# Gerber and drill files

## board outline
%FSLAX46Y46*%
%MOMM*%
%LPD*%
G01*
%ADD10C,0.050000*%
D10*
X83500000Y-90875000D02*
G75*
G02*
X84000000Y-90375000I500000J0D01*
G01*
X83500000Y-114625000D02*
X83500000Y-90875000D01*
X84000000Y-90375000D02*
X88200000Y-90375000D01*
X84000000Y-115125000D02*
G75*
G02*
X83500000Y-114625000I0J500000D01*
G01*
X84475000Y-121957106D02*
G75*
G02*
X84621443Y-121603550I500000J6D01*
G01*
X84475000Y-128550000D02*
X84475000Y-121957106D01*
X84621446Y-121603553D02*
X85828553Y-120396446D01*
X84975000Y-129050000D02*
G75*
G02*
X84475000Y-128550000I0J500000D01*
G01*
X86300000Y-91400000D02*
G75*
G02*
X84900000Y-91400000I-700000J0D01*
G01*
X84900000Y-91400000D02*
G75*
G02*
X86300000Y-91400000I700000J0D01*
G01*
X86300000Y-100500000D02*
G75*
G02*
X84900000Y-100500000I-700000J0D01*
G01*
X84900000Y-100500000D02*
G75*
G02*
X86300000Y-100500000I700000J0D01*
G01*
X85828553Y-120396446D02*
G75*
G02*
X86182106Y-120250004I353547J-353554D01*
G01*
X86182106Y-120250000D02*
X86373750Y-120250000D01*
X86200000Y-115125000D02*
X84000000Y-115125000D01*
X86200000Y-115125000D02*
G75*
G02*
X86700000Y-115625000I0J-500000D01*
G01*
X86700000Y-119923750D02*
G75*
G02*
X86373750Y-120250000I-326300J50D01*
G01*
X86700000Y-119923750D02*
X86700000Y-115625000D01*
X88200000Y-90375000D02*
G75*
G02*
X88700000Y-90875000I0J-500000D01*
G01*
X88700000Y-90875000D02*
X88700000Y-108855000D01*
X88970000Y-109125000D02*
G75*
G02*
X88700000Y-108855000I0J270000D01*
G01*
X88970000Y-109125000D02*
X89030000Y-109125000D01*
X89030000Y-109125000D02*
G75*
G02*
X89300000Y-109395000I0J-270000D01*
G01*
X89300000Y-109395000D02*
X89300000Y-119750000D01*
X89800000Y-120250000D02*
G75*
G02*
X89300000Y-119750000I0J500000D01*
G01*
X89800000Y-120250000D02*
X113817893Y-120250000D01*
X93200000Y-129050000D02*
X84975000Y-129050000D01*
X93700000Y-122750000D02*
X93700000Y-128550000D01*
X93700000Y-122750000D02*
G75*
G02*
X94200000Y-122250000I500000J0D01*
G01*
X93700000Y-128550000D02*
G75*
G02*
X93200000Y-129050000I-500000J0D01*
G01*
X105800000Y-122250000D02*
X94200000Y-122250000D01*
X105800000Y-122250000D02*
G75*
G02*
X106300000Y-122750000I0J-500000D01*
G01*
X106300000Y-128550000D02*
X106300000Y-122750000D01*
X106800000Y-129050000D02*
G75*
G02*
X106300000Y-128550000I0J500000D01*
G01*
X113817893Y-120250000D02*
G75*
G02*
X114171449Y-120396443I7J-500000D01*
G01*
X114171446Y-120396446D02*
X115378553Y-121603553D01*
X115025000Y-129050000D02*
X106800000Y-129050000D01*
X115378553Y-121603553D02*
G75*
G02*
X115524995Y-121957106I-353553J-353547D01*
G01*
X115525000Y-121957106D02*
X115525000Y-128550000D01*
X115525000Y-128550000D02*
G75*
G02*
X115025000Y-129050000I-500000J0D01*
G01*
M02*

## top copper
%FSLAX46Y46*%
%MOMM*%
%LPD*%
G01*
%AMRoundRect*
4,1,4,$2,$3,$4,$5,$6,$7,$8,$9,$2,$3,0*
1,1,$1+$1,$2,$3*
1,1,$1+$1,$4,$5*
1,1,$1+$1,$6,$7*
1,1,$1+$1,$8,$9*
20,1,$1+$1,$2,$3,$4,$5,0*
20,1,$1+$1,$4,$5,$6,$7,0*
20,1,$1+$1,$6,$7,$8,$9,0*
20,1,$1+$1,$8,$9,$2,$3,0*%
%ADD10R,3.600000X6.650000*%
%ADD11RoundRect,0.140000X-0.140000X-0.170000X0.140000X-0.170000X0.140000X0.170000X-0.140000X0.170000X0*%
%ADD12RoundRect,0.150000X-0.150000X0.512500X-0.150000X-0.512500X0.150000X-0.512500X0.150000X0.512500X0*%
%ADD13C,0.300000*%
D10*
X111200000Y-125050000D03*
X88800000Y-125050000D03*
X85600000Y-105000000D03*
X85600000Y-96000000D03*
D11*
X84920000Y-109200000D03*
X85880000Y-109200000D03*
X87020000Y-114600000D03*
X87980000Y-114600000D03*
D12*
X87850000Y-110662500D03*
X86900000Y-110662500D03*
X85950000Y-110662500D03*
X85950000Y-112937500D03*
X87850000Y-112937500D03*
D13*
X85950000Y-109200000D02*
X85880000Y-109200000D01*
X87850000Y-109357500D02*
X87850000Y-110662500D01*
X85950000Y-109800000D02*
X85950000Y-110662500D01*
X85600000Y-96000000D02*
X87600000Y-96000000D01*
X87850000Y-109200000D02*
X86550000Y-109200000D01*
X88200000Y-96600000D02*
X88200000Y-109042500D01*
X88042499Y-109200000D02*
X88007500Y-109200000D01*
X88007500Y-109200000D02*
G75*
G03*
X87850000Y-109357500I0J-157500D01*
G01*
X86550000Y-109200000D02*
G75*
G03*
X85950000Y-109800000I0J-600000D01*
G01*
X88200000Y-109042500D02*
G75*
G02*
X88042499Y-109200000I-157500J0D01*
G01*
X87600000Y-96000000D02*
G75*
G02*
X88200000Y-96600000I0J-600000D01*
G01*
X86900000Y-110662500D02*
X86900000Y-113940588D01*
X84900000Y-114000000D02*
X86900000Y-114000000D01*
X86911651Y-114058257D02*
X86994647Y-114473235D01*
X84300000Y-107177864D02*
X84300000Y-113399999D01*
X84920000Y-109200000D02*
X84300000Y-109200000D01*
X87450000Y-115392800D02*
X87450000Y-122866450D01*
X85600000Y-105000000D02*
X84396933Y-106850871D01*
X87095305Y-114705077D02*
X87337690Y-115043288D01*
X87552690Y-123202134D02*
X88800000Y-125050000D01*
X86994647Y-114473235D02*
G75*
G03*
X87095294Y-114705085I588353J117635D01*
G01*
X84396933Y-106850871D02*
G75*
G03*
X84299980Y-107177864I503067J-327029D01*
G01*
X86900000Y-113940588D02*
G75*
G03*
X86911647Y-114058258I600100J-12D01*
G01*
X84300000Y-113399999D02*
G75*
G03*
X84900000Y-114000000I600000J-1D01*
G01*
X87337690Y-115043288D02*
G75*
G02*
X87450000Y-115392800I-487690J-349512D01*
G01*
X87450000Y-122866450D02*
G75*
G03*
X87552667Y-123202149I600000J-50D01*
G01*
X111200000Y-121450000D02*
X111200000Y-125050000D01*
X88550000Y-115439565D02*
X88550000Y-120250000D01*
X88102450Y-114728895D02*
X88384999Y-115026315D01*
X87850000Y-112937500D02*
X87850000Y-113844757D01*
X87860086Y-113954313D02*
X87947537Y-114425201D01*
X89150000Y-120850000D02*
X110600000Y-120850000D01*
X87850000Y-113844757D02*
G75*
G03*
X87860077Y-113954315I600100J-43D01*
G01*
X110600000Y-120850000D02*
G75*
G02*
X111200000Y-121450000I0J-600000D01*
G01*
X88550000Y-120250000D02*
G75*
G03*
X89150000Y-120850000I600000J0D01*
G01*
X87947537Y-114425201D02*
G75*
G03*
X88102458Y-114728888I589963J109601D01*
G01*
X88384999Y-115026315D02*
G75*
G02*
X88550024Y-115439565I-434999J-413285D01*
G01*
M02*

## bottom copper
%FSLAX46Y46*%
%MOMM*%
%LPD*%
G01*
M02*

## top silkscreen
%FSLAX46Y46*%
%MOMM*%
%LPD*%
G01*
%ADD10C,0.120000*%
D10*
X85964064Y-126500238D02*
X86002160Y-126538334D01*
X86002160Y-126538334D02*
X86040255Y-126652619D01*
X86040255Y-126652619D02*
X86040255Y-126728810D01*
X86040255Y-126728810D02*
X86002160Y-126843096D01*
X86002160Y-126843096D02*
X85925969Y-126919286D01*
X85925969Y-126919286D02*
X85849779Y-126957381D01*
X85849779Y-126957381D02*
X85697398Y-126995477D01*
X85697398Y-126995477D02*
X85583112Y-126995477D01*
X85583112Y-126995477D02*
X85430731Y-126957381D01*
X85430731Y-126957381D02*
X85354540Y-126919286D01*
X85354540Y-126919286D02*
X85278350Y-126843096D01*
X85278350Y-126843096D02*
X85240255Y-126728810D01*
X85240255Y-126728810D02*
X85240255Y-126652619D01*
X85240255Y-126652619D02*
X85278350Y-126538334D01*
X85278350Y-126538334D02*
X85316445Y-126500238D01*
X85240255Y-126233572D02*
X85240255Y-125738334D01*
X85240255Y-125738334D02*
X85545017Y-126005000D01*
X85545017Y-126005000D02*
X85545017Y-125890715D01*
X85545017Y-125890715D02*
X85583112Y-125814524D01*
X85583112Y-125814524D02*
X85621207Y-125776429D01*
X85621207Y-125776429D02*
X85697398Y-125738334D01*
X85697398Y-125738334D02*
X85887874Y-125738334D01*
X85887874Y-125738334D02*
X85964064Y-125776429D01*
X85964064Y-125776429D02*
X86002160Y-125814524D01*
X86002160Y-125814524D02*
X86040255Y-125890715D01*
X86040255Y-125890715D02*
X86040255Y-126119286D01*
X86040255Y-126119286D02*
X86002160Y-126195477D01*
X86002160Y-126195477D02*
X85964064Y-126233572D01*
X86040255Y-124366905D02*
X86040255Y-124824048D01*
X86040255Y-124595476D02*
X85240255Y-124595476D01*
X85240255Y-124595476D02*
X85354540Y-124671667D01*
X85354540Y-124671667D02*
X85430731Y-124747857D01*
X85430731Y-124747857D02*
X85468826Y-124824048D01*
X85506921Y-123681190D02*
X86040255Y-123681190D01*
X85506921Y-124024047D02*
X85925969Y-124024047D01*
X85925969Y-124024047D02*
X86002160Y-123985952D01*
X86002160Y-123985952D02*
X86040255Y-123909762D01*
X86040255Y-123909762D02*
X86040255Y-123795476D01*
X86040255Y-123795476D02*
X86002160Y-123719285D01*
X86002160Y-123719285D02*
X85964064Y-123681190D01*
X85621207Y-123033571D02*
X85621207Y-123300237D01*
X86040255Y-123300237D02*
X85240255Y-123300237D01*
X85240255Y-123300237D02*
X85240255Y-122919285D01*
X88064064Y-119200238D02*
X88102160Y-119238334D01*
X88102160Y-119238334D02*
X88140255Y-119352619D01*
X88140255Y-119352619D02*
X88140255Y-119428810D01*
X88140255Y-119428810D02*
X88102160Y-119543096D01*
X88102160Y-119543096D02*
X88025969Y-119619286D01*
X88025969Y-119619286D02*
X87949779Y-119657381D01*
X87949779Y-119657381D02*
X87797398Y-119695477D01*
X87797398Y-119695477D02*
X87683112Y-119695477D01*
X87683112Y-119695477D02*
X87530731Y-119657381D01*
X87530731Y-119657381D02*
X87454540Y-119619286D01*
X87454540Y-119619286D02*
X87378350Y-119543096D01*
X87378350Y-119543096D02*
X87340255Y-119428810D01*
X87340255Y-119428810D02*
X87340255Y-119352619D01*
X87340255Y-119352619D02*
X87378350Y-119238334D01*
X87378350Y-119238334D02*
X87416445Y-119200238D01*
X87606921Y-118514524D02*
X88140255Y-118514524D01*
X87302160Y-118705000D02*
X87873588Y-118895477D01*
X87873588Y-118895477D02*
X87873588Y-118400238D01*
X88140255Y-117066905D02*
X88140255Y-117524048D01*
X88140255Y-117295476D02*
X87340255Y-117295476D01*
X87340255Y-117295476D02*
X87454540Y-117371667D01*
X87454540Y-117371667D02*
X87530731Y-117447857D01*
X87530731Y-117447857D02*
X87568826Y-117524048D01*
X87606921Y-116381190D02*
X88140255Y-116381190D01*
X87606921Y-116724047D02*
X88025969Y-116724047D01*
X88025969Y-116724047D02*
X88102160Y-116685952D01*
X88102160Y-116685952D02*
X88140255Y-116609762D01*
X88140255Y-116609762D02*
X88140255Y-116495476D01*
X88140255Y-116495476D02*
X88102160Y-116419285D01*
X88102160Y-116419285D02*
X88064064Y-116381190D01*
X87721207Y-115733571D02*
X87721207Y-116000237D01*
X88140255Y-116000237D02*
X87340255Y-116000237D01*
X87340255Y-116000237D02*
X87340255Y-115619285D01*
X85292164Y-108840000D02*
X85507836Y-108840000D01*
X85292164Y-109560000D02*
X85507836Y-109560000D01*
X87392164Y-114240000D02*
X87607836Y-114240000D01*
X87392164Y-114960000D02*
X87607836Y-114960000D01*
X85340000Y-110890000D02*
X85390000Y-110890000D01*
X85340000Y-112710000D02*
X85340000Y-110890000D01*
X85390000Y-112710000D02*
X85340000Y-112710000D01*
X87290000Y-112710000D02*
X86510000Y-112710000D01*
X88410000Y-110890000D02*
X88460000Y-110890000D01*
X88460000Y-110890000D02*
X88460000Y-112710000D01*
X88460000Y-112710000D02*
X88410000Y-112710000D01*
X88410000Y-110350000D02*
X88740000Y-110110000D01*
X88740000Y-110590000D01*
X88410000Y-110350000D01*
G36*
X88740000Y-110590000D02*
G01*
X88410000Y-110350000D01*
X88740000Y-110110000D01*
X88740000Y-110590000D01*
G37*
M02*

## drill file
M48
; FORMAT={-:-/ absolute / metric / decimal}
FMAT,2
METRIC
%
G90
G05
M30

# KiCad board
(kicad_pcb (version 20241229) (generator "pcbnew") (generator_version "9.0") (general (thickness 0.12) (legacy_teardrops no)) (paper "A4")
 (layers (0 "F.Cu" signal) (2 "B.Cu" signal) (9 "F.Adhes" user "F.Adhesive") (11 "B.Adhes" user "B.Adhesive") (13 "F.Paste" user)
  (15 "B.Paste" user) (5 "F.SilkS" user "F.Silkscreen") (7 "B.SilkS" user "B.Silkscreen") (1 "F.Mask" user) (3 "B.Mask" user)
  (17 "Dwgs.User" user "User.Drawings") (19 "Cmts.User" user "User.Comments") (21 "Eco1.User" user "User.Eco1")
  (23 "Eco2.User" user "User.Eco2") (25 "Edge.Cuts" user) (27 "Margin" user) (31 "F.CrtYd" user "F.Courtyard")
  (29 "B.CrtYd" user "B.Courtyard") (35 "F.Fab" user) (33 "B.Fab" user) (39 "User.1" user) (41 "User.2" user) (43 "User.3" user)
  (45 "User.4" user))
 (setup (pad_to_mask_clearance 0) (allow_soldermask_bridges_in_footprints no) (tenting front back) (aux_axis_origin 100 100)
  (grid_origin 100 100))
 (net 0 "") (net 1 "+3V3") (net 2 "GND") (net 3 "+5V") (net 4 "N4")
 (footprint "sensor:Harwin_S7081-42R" (layer "F.Cu") (at 111.2 125.05 90)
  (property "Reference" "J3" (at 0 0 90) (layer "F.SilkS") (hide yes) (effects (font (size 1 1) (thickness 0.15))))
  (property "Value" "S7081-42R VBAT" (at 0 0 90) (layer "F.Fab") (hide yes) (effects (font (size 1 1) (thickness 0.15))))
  (pad "1" smd rect (at 0 0 90) (size 6.65 3.6) (layers "F.Cu" "F.Mask" "F.Paste") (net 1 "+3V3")))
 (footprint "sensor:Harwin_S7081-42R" (layer "F.Cu") (at 88.8 125.05 90)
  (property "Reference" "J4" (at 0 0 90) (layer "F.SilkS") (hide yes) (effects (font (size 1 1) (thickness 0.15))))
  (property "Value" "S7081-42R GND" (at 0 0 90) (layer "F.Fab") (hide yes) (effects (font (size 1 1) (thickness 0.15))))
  (pad "1" smd rect (at 0 0 90) (size 6.65 3.6) (layers "F.Cu" "F.Mask" "F.Paste") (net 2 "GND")))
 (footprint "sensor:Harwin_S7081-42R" (layer "F.Cu") (at 85.6 105 90)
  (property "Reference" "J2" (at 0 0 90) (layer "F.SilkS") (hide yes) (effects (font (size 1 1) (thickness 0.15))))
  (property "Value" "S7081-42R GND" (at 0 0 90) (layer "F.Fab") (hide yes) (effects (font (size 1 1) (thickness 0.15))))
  (pad "1" smd rect (at 0 0 90) (size 6.65 3.6) (layers "F.Cu" "F.Mask" "F.Paste") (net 2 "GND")))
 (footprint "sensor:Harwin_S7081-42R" (layer "F.Cu") (at 85.6 96 90)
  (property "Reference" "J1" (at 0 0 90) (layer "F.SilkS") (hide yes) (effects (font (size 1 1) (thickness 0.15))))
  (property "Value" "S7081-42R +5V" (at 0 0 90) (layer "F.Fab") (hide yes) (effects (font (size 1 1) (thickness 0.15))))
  (pad "1" smd rect (at 0 0 90) (size 6.65 3.6) (layers "F.Cu" "F.Mask" "F.Paste") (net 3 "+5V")))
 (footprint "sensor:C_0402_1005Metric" (layer "F.Cu") (at 85.4 109.2)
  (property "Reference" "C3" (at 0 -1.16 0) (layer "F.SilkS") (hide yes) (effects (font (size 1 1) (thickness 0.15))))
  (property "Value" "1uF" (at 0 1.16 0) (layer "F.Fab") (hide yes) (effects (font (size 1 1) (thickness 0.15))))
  (fp_line (start -0.107836 -0.36) (end 0.107836 -0.36) (stroke (width 0.12) (type solid)) (layer "F.SilkS"))
  (fp_line (start -0.107836 0.36) (end 0.107836 0.36) (stroke (width 0.12) (type solid)) (layer "F.SilkS"))
  (pad "1" smd roundrect (at -0.48 0) (size 0.56 0.62) (layers "F.Cu" "F.Mask" "F.Paste") (roundrect_rratio 0.25) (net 2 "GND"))
  (pad "2" smd roundrect (at 0.48 0) (size 0.56 0.62) (layers "F.Cu" "F.Mask" "F.Paste") (roundrect_rratio 0.25) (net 3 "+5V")))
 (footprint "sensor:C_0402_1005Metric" (layer "F.Cu") (at 87.5 114.6)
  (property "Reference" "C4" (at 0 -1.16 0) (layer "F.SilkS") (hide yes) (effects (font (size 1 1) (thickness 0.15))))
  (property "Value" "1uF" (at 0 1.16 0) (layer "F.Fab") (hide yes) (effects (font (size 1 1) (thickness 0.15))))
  (fp_line (start -0.107836 -0.36) (end 0.107836 -0.36) (stroke (width 0.12) (type solid)) (layer "F.SilkS"))
  (fp_line (start -0.107836 0.36) (end 0.107836 0.36) (stroke (width 0.12) (type solid)) (layer "F.SilkS"))
  (pad "1" smd roundrect (at -0.48 0) (size 0.56 0.62) (layers "F.Cu" "F.Mask" "F.Paste") (roundrect_rratio 0.25) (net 2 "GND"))
  (pad "2" smd roundrect (at 0.48 0) (size 0.56 0.62) (layers "F.Cu" "F.Mask" "F.Paste") (roundrect_rratio 0.25) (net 1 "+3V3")))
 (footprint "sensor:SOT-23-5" (layer "F.Cu") (at 86.9 111.8 -90)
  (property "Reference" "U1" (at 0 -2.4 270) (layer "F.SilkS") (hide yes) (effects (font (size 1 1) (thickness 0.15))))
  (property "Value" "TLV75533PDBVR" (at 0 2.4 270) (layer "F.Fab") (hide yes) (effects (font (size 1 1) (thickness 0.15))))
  (fp_line (start -0.91 1.56) (end -0.91 1.51) (stroke (width 0.12) (type solid)) (layer "F.SilkS"))
  (fp_line (start 0.91 1.56) (end -0.91 1.56) (stroke (width 0.12) (type solid)) (layer "F.SilkS"))
  (fp_line (start 0.91 1.51) (end 0.91 1.56) (stroke (width 0.12) (type solid)) (layer "F.SilkS"))
  (fp_line (start 0.91 -0.39) (end 0.91 0.39) (stroke (width 0.12) (type solid)) (layer "F.SilkS"))
  (fp_line (start -0.91 -1.51) (end -0.91 -1.56) (stroke (width 0.12) (type solid)) (layer "F.SilkS"))
  (fp_line (start -0.91 -1.56) (end 0.91 -1.56) (stroke (width 0.12) (type solid)) (layer "F.SilkS"))
  (fp_line (start 0.91 -1.56) (end 0.91 -1.51) (stroke (width 0.12) (type solid)) (layer "F.SilkS"))
  (fp_poly (pts (xy -1.45 -1.51) (xy -1.69 -1.84) (xy -1.21 -1.84)) (stroke (width 0.12) (type solid)) (fill yes) (layer "F.SilkS"))
  (pad "1" smd roundrect (at -1.1375 -0.95 270) (size 1.325 0.6) (layers "F.Cu" "F.Mask" "F.Paste") (roundrect_rratio 0.25) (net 3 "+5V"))
  (pad "2" smd roundrect (at -1.1375 0 270) (size 1.325 0.6) (layers "F.Cu" "F.Mask" "F.Paste") (roundrect_rratio 0.25) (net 2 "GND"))
  (pad "3" smd roundrect (at -1.1375 0.95 270) (size 1.325 0.6) (layers "F.Cu" "F.Mask" "F.Paste") (roundrect_rratio 0.25) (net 3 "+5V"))
  (pad "4" smd roundrect (at 1.1375 0.95 270) (size 1.325 0.6) (layers "F.Cu" "F.Mask" "F.Paste") (roundrect_rratio 0.25) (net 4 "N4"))
  (pad "5" smd roundrect (at 1.1375 -0.95 270) (size 1.325 0.6) (layers "F.Cu" "F.Mask" "F.Paste") (roundrect_rratio 0.25) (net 1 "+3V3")))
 (gr_arc (start 83.5 90.875) (mid 83.646446 90.521446) (end 84 90.375) (stroke (width 0.05) (type default)) (layer "Edge.Cuts"))
 (gr_line (start 83.5 114.625) (end 83.5 90.875) (stroke (width 0.05) (type default)) (layer "Edge.Cuts"))
 (gr_line (start 84 90.375) (end 88.2 90.375) (stroke (width 0.05) (type default)) (layer "Edge.Cuts"))
 (gr_arc (start 84 115.125) (mid 83.646446 114.978553) (end 83.5 114.625) (stroke (width 0.05) (type default)) (layer "Edge.Cuts"))
 (gr_arc (start 84.475 121.957106) (mid 84.51306 121.765765) (end 84.621446 121.603553) (stroke (width 0.05) (type default))
  (layer "Edge.Cuts"))
 (gr_line (start 84.475 128.55) (end 84.475 121.957106) (stroke (width 0.05) (type default)) (layer "Edge.Cuts"))
 (gr_line (start 84.621446 121.603553) (end 85.828553 120.396446) (stroke (width 0.05) (type default)) (layer "Edge.Cuts"))
 (gr_arc (start 84.975 129.05) (mid 84.621446 128.903553) (end 84.475 128.55) (stroke (width 0.05) (type default)) (layer "Edge.Cuts"))
 (gr_circle (center 85.6 91.4) (end 86.3 91.4) (stroke (width 0.05) (type default)) (fill no) (layer "Edge.Cuts"))
 (gr_circle (center 85.6 100.5) (end 86.3 100.5) (stroke (width 0.05) (type default)) (fill no) (layer "Edge.Cuts"))
 (gr_arc (start 85.828553 120.396446) (mid 85.990765 120.28806) (end 86.182106 120.25) (stroke (width 0.05) (type default))
  (layer "Edge.Cuts"))
 (gr_line (start 86.182106 120.25) (end 86.37375 120.25) (stroke (width 0.05) (type default)) (layer "Edge.Cuts"))
 (gr_line (start 86.2 115.125) (end 84 115.125) (stroke (width 0.05) (type default)) (layer "Edge.Cuts"))
 (gr_arc (start 86.2 115.125) (mid 86.553553 115.271447) (end 86.7 115.625) (stroke (width 0.05) (type default)) (layer "Edge.Cuts"))
 (gr_arc (start 86.7 119.92375) (mid 86.604429 120.154429) (end 86.37375 120.25) (stroke (width 0.05) (type default)) (layer "Edge.Cuts"))
 (gr_line (start 86.7 119.92375) (end 86.7 115.625) (stroke (width 0.05) (type default)) (layer "Edge.Cuts"))
 (gr_arc (start 88.2 90.375) (mid 88.553553 90.521446) (end 88.7 90.875) (stroke (width 0.05) (type default)) (layer "Edge.Cuts"))
 (gr_line (start 88.7 90.875) (end 88.7 108.855) (stroke (width 0.05) (type default)) (layer "Edge.Cuts"))
 (gr_arc (start 88.97 109.125) (mid 88.779081 109.045919) (end 88.7 108.855) (stroke (width 0.05) (type default)) (layer "Edge.Cuts"))
 (gr_line (start 88.97 109.125) (end 89.03 109.125) (stroke (width 0.05) (type default)) (layer "Edge.Cuts"))
 (gr_arc (start 89.03 109.125) (mid 89.220918 109.204081) (end 89.3 109.395) (stroke (width 0.05) (type default)) (layer "Edge.Cuts"))
 (gr_line (start 89.3 109.395) (end 89.3 119.75) (stroke (width 0.05) (type default)) (layer "Edge.Cuts"))
 (gr_arc (start 89.8 120.25) (mid 89.446447 120.103553) (end 89.3 119.75) (stroke (width 0.05) (type default)) (layer "Edge.Cuts"))
 (gr_line (start 89.8 120.25) (end 113.817893 120.25) (stroke (width 0.05) (type default)) (layer "Edge.Cuts"))
 (gr_line (start 93.2 129.05) (end 84.975 129.05) (stroke (width 0.05) (type default)) (layer "Edge.Cuts"))
 (gr_line (start 93.7 122.75) (end 93.7 128.55) (stroke (width 0.05) (type default)) (layer "Edge.Cuts"))
 (gr_arc (start 93.7 122.75) (mid 93.846447 122.396447) (end 94.2 122.25) (stroke (width 0.05) (type default)) (layer "Edge.Cuts"))
 (gr_arc (start 93.7 128.55) (mid 93.553553 128.903553) (end 93.2 129.05) (stroke (width 0.05) (type default)) (layer "Edge.Cuts"))
 (gr_line (start 105.8 122.25) (end 94.2 122.25) (stroke (width 0.05) (type default)) (layer "Edge.Cuts"))
 (gr_arc (start 105.8 122.25) (mid 106.153553 122.396447) (end 106.3 122.75) (stroke (width 0.05) (type default)) (layer "Edge.Cuts"))
 (gr_line (start 106.3 128.55) (end 106.3 122.75) (stroke (width 0.05) (type default)) (layer "Edge.Cuts"))
 (gr_arc (start 106.8 129.05) (mid 106.446446 128.903553) (end 106.3 128.55) (stroke (width 0.05) (type default)) (layer "Edge.Cuts"))
 (gr_arc (start 113.817893 120.25) (mid 114.009234 120.28806) (end 114.171446 120.396446) (stroke (width 0.05) (type default))
  (layer "Edge.Cuts"))
 (gr_line (start 114.171446 120.396446) (end 115.378553 121.603553) (stroke (width 0.05) (type default)) (layer "Edge.Cuts"))
 (gr_line (start 115.025 129.05) (end 106.8 129.05) (stroke (width 0.05) (type default)) (layer "Edge.Cuts"))
 (gr_arc (start 115.378553 121.603553) (mid 115.486939 121.765765) (end 115.525 121.957106) (stroke (width 0.05) (type default))
  (layer "Edge.Cuts"))
 (gr_line (start 115.525 121.957106) (end 115.525 128.55) (stroke (width 0.05) (type default)) (layer "Edge.Cuts"))
 (gr_arc (start 115.525 128.55) (mid 115.378553 128.903553) (end 115.025 129.05) (stroke (width 0.05) (type default)) (layer "Edge.Cuts"))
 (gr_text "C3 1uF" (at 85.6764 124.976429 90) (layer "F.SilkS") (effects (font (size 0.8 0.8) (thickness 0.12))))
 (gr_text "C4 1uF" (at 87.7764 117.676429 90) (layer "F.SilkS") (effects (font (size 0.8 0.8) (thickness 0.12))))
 (segment (start 85.95 109.2) (end 85.88 109.2) (width 0.3) (layer "F.Cu") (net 3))
 (segment (start 87.85 109.3575) (end 87.85 110.6625) (width 0.3) (layer "F.Cu") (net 3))
 (segment (start 85.95 109.8) (end 85.95 110.6625) (width 0.3) (layer "F.Cu") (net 3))
 (segment (start 85.6 96) (end 87.6 96) (width 0.3) (layer "F.Cu") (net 3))
 (segment (start 87.85 109.2) (end 86.55 109.2) (width 0.3) (layer "F.Cu") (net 3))
 (segment (start 88.2 96.6) (end 88.2 109.0425) (width 0.3) (layer "F.Cu") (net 3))
 (segment (start 88.042499 109.2) (end 88.0075 109.2) (width 0.3) (layer "F.Cu") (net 3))
 (arc (start 88.0075 109.2) (mid 87.89613 109.24613) (end 87.85 109.3575) (width 0.3) (layer "F.Cu") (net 3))
 (arc (start 86.55 109.2) (mid 86.125735 109.375735) (end 85.95 109.8) (width 0.3) (layer "F.Cu") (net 3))
 (arc (start 88.2 109.0425) (mid 88.153869 109.153869) (end 88.042499 109.2) (width 0.3) (layer "F.Cu") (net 3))
 (arc (start 87.6 96) (mid 88.024264 96.175735) (end 88.2 96.6) (width 0.3) (layer "F.Cu") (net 3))
 (segment (start 86.9 110.6625) (end 86.9 113.940588) (width 0.3) (layer "F.Cu") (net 2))
 (segment (start 84.9 114) (end 86.9 114) (width 0.3) (layer "F.Cu") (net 2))
 (segment (start 86.911651 114.058257) (end 86.994647 114.473235) (width 0.3) (layer "F.Cu") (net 2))
 (segment (start 84.3 107.177864) (end 84.3 113.399999) (width 0.3) (layer "F.Cu") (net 2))
 (segment (start 84.92 109.2) (end 84.3 109.2) (width 0.3) (layer "F.Cu") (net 2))
 (segment (start 87.45 115.3928) (end 87.45 122.86645) (width 0.3) (layer "F.Cu") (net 2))
 (segment (start 85.6 105) (end 84.396933 106.850871) (width 0.3) (layer "F.Cu") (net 2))
 (segment (start 87.095305 114.705077) (end 87.33769 115.043288) (width 0.3) (layer "F.Cu") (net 2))
 (segment (start 87.55269 123.202134) (end 88.8 125.05) (width 0.3) (layer "F.Cu") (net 2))
 (arc (start 86.994647 114.473235) (mid 87.032629 114.594516) (end 87.095305 114.705077) (width 0.3) (layer "F.Cu") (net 2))
 (arc (start 84.396933 106.850871) (mid 84.324743 107.007335) (end 84.3 107.177864) (width 0.3) (layer "F.Cu") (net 2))
 (arc (start 86.9 113.940588) (mid 86.90292 113.99971) (end 86.911651 114.058257) (width 0.3) (layer "F.Cu") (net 2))
 (arc (start 84.3 113.399999) (mid 84.475735 113.824264) (end 84.9 114) (width 0.3) (layer "F.Cu") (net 2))
 (arc (start 87.33769 115.043288) (mid 87.421232 115.209243) (end 87.45 115.3928) (width 0.3) (layer "F.Cu") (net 2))
 (arc (start 87.45 122.86645) (mid 87.476246 123.04197) (end 87.55269 123.202134) (width 0.3) (layer "F.Cu") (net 2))
 (segment (start 111.2 121.45) (end 111.2 125.05) (width 0.3) (layer "F.Cu") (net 1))
 (segment (start 88.55 115.439565) (end 88.55 120.25) (width 0.3) (layer "F.Cu") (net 1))
 (segment (start 88.10245 114.728895) (end 88.384999 115.026315) (width 0.3) (layer "F.Cu") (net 1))
 (segment (start 87.85 112.9375) (end 87.85 113.844757) (width 0.3) (layer "F.Cu") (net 1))
 (segment (start 87.860086 113.954313) (end 87.947537 114.425201) (width 0.3) (layer "F.Cu") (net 1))
 (segment (start 89.15 120.85) (end 110.6 120.85) (width 0.3) (layer "F.Cu") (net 1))
 (arc (start 87.85 113.844757) (mid 87.852527 113.899767) (end 87.860086 113.954313) (width 0.3) (layer "F.Cu") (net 1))
 (arc (start 110.6 120.85) (mid 111.024264 121.025735) (end 111.2 121.45) (width 0.3) (layer "F.Cu") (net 1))
 (arc (start 88.55 120.25) (mid 88.725735 120.674264) (end 89.15 120.85) (width 0.3) (layer "F.Cu") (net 1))
 (arc (start 87.947537 114.425201) (mid 88.00297 114.588282) (end 88.10245 114.728895) (width 0.3) (layer "F.Cu") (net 1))
 (arc (start 88.384999 115.026315) (mid 88.507225 115.217078) (end 88.55 115.439565) (width 0.3) (layer "F.Cu") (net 1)))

